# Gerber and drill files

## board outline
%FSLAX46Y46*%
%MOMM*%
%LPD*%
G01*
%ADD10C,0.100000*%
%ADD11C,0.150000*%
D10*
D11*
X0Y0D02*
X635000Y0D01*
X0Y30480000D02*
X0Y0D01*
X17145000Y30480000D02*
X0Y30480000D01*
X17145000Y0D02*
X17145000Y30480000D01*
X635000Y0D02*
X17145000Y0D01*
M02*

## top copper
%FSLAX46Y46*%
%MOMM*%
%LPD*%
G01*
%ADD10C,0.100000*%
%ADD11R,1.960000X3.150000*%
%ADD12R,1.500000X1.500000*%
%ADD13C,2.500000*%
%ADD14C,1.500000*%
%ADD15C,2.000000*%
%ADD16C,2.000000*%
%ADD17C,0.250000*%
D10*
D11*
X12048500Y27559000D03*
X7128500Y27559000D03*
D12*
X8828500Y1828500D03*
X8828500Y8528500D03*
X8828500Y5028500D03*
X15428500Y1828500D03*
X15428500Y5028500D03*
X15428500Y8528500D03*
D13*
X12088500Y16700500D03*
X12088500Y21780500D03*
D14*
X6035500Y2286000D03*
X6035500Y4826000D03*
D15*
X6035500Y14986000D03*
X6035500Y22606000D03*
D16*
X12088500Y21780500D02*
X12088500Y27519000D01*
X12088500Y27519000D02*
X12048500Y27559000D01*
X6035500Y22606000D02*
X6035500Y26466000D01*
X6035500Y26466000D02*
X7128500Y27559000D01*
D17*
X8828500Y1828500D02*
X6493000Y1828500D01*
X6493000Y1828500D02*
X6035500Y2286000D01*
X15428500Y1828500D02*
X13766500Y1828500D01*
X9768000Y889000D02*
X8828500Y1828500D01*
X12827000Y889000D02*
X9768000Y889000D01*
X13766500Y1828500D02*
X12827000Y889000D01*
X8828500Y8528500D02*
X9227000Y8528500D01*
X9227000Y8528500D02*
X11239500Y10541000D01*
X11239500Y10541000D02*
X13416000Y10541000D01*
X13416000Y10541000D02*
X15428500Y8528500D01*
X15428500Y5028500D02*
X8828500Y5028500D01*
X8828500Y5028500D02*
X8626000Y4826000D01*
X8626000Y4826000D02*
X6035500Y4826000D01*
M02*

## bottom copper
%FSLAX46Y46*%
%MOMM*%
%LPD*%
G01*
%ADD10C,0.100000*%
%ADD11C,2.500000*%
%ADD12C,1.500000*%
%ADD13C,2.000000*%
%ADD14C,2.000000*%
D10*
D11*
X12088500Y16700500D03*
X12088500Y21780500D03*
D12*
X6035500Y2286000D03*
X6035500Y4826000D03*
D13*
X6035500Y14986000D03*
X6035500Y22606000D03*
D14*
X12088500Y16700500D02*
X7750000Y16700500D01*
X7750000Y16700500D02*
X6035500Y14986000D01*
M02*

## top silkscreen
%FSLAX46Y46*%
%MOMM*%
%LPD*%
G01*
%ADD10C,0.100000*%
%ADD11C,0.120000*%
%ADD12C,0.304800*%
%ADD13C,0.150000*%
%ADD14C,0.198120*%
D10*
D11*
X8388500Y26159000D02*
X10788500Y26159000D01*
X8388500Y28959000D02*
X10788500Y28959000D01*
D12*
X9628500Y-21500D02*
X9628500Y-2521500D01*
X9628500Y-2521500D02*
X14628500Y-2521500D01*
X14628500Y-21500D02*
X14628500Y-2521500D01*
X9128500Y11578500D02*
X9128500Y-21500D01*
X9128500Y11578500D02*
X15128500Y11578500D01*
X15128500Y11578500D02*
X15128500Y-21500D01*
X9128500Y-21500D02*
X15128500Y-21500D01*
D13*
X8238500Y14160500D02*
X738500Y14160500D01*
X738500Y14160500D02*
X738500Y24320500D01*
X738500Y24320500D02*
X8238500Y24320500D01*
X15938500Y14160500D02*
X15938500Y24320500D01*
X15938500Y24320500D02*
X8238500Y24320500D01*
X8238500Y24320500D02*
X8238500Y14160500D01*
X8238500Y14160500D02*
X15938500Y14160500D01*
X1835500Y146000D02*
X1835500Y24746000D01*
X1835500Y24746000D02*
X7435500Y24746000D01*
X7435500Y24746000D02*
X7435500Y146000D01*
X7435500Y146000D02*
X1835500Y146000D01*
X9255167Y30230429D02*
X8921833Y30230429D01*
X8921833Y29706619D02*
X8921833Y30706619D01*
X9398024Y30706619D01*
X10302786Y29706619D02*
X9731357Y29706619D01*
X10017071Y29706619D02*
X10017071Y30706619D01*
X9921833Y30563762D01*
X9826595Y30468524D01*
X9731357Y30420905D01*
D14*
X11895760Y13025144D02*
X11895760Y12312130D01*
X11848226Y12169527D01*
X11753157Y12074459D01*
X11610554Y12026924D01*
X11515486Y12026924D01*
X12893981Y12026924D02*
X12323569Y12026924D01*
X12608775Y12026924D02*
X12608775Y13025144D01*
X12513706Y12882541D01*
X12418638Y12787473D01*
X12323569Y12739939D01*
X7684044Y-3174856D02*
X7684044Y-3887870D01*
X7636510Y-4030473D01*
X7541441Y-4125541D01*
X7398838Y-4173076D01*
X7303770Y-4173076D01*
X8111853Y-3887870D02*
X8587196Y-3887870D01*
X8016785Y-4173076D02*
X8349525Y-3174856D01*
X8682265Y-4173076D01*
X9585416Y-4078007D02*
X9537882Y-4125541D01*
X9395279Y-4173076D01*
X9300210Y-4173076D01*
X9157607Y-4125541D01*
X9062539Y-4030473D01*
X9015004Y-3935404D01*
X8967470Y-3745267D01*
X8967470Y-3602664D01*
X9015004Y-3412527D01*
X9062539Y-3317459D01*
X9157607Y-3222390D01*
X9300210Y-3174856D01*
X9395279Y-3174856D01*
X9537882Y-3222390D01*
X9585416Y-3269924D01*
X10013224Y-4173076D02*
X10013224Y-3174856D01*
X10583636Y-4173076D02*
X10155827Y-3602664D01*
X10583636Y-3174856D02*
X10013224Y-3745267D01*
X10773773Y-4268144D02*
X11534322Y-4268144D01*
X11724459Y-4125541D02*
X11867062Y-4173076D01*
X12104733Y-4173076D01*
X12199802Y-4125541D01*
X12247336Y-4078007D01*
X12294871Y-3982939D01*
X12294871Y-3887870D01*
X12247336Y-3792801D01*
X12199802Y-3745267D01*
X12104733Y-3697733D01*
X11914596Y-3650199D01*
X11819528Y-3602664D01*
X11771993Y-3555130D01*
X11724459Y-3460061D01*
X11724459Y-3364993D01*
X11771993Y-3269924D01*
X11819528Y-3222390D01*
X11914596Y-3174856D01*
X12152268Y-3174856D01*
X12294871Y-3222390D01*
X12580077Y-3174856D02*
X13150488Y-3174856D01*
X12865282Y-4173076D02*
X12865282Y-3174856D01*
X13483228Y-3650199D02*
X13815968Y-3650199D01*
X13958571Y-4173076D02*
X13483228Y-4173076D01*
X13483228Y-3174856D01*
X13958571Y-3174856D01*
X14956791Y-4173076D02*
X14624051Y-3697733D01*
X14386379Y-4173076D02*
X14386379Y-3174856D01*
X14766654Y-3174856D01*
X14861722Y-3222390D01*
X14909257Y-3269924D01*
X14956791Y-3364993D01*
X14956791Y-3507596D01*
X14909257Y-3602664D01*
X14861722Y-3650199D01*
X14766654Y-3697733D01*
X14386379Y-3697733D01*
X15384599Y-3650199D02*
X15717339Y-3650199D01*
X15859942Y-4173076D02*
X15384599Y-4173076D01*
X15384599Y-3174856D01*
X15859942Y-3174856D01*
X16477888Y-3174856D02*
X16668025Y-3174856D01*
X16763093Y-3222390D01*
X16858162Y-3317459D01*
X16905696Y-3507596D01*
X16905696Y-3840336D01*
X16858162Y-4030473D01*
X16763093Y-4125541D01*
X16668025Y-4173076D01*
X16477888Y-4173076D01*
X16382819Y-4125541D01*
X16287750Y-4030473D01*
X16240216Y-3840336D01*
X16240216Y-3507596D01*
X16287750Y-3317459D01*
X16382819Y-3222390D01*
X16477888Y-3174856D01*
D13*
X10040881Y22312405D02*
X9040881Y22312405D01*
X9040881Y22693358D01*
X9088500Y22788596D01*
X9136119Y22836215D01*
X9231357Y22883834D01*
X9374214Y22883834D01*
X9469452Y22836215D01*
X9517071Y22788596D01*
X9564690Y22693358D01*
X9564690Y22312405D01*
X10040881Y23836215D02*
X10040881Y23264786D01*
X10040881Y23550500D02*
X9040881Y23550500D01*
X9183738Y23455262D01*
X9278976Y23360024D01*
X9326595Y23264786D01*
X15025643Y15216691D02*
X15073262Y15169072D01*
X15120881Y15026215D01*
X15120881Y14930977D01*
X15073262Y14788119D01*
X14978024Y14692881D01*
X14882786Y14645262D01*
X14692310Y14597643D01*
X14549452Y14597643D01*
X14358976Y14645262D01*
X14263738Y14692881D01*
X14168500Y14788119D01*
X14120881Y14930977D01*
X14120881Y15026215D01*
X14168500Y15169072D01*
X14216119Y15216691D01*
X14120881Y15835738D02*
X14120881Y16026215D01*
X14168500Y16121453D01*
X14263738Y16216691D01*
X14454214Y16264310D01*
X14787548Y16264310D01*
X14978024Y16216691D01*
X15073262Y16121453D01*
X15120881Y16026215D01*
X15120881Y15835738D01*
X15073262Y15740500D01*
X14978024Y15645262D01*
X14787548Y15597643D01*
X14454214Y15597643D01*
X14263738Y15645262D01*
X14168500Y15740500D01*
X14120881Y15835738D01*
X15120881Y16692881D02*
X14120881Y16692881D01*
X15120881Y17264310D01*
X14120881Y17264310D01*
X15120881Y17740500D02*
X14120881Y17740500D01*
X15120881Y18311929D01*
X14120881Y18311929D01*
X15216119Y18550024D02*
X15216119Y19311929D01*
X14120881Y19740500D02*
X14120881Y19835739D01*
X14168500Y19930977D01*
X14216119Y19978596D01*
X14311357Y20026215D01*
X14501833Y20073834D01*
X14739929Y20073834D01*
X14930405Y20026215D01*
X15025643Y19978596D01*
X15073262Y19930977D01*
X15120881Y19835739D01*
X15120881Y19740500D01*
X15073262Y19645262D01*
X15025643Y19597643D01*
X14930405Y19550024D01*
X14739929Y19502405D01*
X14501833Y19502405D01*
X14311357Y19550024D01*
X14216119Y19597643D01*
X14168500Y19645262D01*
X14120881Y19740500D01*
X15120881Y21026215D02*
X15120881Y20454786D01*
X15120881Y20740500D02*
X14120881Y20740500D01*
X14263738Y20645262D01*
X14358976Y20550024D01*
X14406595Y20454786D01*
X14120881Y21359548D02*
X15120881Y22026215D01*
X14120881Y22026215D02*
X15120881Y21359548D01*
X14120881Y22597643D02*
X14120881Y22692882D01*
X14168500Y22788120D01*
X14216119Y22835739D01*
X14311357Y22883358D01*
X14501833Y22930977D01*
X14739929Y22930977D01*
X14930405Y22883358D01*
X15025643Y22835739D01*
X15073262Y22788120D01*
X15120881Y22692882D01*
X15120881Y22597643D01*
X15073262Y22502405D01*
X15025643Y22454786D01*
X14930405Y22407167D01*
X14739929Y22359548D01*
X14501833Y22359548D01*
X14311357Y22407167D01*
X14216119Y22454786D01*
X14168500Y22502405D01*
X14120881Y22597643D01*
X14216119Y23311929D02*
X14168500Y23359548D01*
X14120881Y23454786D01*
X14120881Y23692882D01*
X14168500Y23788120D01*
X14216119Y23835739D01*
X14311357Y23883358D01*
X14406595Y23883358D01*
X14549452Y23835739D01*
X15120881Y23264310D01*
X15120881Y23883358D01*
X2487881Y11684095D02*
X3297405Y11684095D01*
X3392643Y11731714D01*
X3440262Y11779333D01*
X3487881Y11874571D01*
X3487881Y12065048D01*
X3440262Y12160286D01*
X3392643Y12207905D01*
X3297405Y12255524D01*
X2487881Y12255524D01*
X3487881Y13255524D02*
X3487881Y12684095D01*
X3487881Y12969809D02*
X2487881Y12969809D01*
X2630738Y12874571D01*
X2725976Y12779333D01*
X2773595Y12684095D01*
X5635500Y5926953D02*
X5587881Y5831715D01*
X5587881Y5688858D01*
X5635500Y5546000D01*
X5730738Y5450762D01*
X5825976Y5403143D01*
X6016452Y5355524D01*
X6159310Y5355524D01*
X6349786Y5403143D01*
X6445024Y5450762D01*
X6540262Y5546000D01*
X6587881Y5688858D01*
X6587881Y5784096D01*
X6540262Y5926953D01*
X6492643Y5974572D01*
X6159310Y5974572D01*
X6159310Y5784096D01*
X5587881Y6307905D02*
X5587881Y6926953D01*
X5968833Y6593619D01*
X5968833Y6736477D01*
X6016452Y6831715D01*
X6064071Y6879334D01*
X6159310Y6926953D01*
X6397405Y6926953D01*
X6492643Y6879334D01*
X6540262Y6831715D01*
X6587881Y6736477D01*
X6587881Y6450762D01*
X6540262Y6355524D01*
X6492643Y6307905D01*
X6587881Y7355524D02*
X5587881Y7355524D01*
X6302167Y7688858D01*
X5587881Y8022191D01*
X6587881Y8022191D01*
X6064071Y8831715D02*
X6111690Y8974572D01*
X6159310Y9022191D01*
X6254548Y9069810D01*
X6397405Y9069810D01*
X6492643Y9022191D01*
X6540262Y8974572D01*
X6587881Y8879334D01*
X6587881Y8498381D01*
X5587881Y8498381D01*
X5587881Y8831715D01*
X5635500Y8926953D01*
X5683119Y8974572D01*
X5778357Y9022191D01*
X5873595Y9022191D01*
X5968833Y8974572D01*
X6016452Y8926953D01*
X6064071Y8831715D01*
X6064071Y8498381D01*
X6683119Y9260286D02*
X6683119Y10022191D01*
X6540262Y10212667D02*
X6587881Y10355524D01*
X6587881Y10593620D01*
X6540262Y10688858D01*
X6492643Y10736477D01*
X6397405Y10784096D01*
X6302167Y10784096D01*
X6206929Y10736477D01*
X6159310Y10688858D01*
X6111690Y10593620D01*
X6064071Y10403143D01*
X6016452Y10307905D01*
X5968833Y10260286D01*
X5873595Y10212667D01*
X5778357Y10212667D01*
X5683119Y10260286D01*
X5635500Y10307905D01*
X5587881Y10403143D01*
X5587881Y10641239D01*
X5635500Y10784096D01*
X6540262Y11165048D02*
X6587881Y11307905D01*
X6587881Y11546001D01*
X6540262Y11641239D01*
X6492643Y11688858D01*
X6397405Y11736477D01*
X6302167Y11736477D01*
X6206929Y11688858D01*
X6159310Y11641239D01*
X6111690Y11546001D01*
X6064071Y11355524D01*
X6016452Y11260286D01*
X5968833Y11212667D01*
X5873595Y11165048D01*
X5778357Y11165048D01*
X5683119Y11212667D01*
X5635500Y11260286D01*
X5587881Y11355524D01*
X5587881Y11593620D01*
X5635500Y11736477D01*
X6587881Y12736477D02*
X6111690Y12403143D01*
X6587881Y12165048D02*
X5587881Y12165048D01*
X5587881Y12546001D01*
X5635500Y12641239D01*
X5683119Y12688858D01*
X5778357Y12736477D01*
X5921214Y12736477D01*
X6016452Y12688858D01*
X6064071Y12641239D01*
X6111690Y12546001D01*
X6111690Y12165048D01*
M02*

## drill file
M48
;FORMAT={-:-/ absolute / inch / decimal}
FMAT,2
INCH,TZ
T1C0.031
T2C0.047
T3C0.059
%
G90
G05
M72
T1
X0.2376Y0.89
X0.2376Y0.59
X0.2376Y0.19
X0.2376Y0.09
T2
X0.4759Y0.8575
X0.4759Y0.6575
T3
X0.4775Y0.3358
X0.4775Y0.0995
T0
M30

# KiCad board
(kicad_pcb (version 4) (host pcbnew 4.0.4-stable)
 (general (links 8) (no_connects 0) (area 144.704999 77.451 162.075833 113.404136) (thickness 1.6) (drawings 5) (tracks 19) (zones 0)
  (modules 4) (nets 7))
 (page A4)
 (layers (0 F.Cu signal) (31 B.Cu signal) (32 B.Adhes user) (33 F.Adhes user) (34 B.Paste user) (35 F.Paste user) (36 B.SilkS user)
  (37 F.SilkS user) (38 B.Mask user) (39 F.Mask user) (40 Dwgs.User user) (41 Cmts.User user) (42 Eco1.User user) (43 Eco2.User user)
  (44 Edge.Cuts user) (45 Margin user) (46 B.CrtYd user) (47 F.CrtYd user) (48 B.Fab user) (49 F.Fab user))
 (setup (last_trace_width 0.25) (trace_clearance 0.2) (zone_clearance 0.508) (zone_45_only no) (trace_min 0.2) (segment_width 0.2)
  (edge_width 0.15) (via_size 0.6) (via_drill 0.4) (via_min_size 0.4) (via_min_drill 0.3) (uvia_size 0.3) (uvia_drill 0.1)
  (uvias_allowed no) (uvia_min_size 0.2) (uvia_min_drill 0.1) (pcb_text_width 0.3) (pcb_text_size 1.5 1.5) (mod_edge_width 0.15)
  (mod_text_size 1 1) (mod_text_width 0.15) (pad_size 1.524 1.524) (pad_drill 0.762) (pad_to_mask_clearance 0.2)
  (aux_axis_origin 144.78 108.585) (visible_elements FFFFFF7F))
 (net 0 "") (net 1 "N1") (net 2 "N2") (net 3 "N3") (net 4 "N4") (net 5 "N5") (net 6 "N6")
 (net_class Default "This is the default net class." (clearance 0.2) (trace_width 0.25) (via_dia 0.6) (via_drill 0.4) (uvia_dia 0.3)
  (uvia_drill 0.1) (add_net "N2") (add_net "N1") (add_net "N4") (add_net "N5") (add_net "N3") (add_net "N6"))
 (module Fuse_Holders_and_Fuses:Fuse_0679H (layer F.Cu) (at 154.3685 81.026)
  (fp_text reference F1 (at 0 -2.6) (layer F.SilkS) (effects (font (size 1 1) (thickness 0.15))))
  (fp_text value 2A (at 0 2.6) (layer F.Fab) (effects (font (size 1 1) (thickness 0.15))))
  (fp_line (start -1.2 1.4) (end 1.2 1.4) (layer F.SilkS) (width 0.12))
  (fp_line (start -1.2 -1.4) (end 1.2 -1.4) (layer F.SilkS) (width 0.12))
  (pad 2 smd rect (at 2.46 0) (size 1.96 3.15) (layers F.Cu F.Paste F.Mask) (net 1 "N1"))
  (pad 1 smd rect (at -2.46 0) (size 1.96 3.15) (layers F.Cu F.Paste F.Mask) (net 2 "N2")))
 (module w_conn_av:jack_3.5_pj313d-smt (layer F.Cu) (at 156.9085 102.8065)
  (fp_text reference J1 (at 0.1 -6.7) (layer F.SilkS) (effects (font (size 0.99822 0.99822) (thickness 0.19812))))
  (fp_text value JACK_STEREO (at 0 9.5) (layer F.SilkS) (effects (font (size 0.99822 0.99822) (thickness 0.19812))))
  (fp_line (start -2.5 5.8) (end -2.5 8.3) (layer F.SilkS) (width 0.3048))
  (fp_line (start -2.5 8.3) (end 2.5 8.3) (layer F.SilkS) (width 0.3048))
  (fp_line (start 2.5 5.8) (end 2.5 8.3) (layer F.SilkS) (width 0.3048))
  (fp_line (start -3 -5.8) (end -3 5.8) (layer F.SilkS) (width 0.3048))
  (fp_line (start -3 -5.8) (end 3 -5.8) (layer F.SilkS) (width 0.3048))
  (fp_line (start 3 -5.8) (end 3 5.8) (layer F.SilkS) (width 0.3048))
  (fp_line (start -3 5.8) (end 3 5.8) (layer F.SilkS) (width 0.3048))
  (pad "" np_thru_hole circle (at 0 3.25) (size 1.5 1.5) (drill 1.5) (layers *.Cu *.Mask F.SilkS))
  (pad "" np_thru_hole circle (at 0 -2.75) (size 1.5 1.5) (drill 1.5) (layers *.Cu *.Mask F.SilkS))
  (pad 3 smd rect (at -3.3 3.95) (size 1.5 1.5) (layers F.Cu F.Paste F.Mask) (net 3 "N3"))
  (pad 1 smd rect (at -3.3 -2.75) (size 1.5 1.5) (layers F.Cu F.Paste F.Mask) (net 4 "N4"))
  (pad 2 smd rect (at -3.3 0.75) (size 1.5 1.5) (layers F.Cu F.Paste F.Mask) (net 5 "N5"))
  (pad 3 smd rect (at 3.3 3.95) (size 1.5 1.5) (layers F.Cu F.Paste F.Mask) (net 3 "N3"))
  (pad 2 smd rect (at 3.3 0.75) (size 1.5 1.5) (layers F.Cu F.Paste F.Mask) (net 5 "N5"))
  (pad 1 smd rect (at 3.3 -2.75) (size 1.5 1.5) (layers F.Cu F.Paste F.Mask) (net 4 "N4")))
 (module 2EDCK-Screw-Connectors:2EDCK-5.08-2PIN (layer F.Cu) (at 160.7185 94.4245 90)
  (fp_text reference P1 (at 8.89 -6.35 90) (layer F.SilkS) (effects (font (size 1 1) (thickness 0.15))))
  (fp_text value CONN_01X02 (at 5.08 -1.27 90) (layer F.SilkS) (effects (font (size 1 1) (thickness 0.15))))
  (fp_line (start 0 -7.7) (end 0 -15.2) (layer F.SilkS) (width 0.15))
  (fp_line (start 0 -15.2) (end 10.16 -15.2) (layer F.SilkS) (width 0.15))
  (fp_line (start 10.16 -15.2) (end 10.16 -7.7) (layer F.SilkS) (width 0.15))
  (fp_line (start 0 0) (end 10.16 0) (layer F.SilkS) (width 0.15))
  (fp_line (start 10.16 0) (end 10.16 -7.7) (layer F.SilkS) (width 0.15))
  (fp_line (start 10.16 -7.7) (end 0 -7.7) (layer F.SilkS) (width 0.15))
  (fp_line (start 0 -7.7) (end 0 0) (layer F.SilkS) (width 0.15))
  (pad 1 thru_hole circle (at 2.54 -3.85 90) (size 2.5 2.5) (drill 1.2) (layers *.Cu *.Mask F.SilkS) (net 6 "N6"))
  (pad 2 thru_hole circle (at 7.62 -3.85 90) (size 2.5 2.5) (drill 1.2) (layers *.Cu *.Mask F.SilkS) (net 1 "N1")))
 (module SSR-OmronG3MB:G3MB (layer F.Cu) (at 149.4155 96.139 90)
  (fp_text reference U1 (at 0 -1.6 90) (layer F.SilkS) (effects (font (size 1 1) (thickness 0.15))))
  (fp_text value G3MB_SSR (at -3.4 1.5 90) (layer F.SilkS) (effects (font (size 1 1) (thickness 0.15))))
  (fp_line (start -12.3 -2.8) (end 12.3 -2.8) (layer F.SilkS) (width 0.15))
  (fp_line (start 12.3 -2.8) (end 12.3 2.8) (layer F.SilkS) (width 0.15))
  (fp_line (start 12.3 2.8) (end -12.3 2.8) (layer F.SilkS) (width 0.15))
  (fp_line (start -12.3 2.8) (end -12.3 -2.8) (layer F.SilkS) (width 0.15))
  (pad 4 thru_hole circle (at -10.16 1.4 90) (size 1.5 1.5) (drill 0.8) (layers *.Cu *.Mask F.SilkS) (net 3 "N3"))
  (pad 3 thru_hole circle (at -7.62 1.4 90) (size 1.5 1.5) (drill 0.8) (layers *.Cu *.Mask F.SilkS) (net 5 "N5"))
  (pad 2 thru_hole circle (at 2.54 1.4 90) (size 2 2) (drill 0.8) (layers *.Cu *.Mask F.SilkS) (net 6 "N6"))
  (pad 1 thru_hole circle (at 10.16 1.4 90) (size 2 2) (drill 0.8) (layers *.Cu *.Mask F.SilkS) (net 2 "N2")))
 (gr_line (start 144.78 108.585) (end 145.415 108.585) (angle 90) (layer Edge.Cuts) (width 0.15))
 (gr_line (start 144.78 78.105) (end 144.78 108.585) (angle 90) (layer Edge.Cuts) (width 0.15))
 (gr_line (start 161.925 78.105) (end 144.78 78.105) (angle 90) (layer Edge.Cuts) (width 0.15))
 (gr_line (start 161.925 108.585) (end 161.925 78.105) (angle 90) (layer Edge.Cuts) (width 0.15))
 (gr_line (start 145.415 108.585) (end 161.925 108.585) (angle 90) (layer Edge.Cuts) (width 0.15))
 (segment (start 156.8685 86.8045) (end 156.8685 81.066) (width 2) (layer F.Cu) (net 1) (status C00000))
 (segment (start 156.8685 81.066) (end 156.8285 81.026) (width 2) (layer F.Cu) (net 1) (status C00000))
 (segment (start 150.8155 85.979) (end 150.8155 82.119) (width 2) (layer F.Cu) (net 2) (status 400000))
 (segment (start 150.8155 82.119) (end 151.9085 81.026) (width 2) (layer F.Cu) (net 2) (status 800000))
 (segment (start 153.6085 106.7565) (end 151.273 106.7565) (width 0.25) (layer F.Cu) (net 3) (status C00000))
 (segment (start 151.273 106.7565) (end 150.8155 106.299) (width 0.25) (layer F.Cu) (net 3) (status C00000))
 (segment (start 160.2085 106.7565) (end 158.5465 106.7565) (width 0.25) (layer F.Cu) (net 3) (status 400000))
 (segment (start 154.548 107.696) (end 153.6085 106.7565) (width 0.25) (layer F.Cu) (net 3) (status 800000))
 (segment (start 157.607 107.696) (end 154.548 107.696) (width 0.25) (layer F.Cu) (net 3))
 (segment (start 158.5465 106.7565) (end 157.607 107.696) (width 0.25) (layer F.Cu) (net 3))
 (segment (start 153.6085 100.0565) (end 154.007 100.0565) (width 0.25) (layer F.Cu) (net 4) (status C00000))
 (segment (start 154.007 100.0565) (end 156.0195 98.044) (width 0.25) (layer F.Cu) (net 4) (status 400000))
 (segment (start 156.0195 98.044) (end 158.196 98.044) (width 0.25) (layer F.Cu) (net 4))
 (segment (start 158.196 98.044) (end 160.2085 100.0565) (width 0.25) (layer F.Cu) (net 4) (status 800000))
 (segment (start 160.2085 103.5565) (end 153.6085 103.5565) (width 0.25) (layer F.Cu) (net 5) (status C00000))
 (segment (start 153.6085 103.5565) (end 153.406 103.759) (width 0.25) (layer F.Cu) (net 5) (status C00000))
 (segment (start 153.406 103.759) (end 150.8155 103.759) (width 0.25) (layer F.Cu) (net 5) (status C00000))
 (segment (start 156.8685 91.8845) (end 152.53 91.8845) (width 2) (layer B.Cu) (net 6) (status 400000))
 (segment (start 152.53 91.8845) (end 150.8155 93.599) (width 2) (layer B.Cu) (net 6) (status 800000)))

